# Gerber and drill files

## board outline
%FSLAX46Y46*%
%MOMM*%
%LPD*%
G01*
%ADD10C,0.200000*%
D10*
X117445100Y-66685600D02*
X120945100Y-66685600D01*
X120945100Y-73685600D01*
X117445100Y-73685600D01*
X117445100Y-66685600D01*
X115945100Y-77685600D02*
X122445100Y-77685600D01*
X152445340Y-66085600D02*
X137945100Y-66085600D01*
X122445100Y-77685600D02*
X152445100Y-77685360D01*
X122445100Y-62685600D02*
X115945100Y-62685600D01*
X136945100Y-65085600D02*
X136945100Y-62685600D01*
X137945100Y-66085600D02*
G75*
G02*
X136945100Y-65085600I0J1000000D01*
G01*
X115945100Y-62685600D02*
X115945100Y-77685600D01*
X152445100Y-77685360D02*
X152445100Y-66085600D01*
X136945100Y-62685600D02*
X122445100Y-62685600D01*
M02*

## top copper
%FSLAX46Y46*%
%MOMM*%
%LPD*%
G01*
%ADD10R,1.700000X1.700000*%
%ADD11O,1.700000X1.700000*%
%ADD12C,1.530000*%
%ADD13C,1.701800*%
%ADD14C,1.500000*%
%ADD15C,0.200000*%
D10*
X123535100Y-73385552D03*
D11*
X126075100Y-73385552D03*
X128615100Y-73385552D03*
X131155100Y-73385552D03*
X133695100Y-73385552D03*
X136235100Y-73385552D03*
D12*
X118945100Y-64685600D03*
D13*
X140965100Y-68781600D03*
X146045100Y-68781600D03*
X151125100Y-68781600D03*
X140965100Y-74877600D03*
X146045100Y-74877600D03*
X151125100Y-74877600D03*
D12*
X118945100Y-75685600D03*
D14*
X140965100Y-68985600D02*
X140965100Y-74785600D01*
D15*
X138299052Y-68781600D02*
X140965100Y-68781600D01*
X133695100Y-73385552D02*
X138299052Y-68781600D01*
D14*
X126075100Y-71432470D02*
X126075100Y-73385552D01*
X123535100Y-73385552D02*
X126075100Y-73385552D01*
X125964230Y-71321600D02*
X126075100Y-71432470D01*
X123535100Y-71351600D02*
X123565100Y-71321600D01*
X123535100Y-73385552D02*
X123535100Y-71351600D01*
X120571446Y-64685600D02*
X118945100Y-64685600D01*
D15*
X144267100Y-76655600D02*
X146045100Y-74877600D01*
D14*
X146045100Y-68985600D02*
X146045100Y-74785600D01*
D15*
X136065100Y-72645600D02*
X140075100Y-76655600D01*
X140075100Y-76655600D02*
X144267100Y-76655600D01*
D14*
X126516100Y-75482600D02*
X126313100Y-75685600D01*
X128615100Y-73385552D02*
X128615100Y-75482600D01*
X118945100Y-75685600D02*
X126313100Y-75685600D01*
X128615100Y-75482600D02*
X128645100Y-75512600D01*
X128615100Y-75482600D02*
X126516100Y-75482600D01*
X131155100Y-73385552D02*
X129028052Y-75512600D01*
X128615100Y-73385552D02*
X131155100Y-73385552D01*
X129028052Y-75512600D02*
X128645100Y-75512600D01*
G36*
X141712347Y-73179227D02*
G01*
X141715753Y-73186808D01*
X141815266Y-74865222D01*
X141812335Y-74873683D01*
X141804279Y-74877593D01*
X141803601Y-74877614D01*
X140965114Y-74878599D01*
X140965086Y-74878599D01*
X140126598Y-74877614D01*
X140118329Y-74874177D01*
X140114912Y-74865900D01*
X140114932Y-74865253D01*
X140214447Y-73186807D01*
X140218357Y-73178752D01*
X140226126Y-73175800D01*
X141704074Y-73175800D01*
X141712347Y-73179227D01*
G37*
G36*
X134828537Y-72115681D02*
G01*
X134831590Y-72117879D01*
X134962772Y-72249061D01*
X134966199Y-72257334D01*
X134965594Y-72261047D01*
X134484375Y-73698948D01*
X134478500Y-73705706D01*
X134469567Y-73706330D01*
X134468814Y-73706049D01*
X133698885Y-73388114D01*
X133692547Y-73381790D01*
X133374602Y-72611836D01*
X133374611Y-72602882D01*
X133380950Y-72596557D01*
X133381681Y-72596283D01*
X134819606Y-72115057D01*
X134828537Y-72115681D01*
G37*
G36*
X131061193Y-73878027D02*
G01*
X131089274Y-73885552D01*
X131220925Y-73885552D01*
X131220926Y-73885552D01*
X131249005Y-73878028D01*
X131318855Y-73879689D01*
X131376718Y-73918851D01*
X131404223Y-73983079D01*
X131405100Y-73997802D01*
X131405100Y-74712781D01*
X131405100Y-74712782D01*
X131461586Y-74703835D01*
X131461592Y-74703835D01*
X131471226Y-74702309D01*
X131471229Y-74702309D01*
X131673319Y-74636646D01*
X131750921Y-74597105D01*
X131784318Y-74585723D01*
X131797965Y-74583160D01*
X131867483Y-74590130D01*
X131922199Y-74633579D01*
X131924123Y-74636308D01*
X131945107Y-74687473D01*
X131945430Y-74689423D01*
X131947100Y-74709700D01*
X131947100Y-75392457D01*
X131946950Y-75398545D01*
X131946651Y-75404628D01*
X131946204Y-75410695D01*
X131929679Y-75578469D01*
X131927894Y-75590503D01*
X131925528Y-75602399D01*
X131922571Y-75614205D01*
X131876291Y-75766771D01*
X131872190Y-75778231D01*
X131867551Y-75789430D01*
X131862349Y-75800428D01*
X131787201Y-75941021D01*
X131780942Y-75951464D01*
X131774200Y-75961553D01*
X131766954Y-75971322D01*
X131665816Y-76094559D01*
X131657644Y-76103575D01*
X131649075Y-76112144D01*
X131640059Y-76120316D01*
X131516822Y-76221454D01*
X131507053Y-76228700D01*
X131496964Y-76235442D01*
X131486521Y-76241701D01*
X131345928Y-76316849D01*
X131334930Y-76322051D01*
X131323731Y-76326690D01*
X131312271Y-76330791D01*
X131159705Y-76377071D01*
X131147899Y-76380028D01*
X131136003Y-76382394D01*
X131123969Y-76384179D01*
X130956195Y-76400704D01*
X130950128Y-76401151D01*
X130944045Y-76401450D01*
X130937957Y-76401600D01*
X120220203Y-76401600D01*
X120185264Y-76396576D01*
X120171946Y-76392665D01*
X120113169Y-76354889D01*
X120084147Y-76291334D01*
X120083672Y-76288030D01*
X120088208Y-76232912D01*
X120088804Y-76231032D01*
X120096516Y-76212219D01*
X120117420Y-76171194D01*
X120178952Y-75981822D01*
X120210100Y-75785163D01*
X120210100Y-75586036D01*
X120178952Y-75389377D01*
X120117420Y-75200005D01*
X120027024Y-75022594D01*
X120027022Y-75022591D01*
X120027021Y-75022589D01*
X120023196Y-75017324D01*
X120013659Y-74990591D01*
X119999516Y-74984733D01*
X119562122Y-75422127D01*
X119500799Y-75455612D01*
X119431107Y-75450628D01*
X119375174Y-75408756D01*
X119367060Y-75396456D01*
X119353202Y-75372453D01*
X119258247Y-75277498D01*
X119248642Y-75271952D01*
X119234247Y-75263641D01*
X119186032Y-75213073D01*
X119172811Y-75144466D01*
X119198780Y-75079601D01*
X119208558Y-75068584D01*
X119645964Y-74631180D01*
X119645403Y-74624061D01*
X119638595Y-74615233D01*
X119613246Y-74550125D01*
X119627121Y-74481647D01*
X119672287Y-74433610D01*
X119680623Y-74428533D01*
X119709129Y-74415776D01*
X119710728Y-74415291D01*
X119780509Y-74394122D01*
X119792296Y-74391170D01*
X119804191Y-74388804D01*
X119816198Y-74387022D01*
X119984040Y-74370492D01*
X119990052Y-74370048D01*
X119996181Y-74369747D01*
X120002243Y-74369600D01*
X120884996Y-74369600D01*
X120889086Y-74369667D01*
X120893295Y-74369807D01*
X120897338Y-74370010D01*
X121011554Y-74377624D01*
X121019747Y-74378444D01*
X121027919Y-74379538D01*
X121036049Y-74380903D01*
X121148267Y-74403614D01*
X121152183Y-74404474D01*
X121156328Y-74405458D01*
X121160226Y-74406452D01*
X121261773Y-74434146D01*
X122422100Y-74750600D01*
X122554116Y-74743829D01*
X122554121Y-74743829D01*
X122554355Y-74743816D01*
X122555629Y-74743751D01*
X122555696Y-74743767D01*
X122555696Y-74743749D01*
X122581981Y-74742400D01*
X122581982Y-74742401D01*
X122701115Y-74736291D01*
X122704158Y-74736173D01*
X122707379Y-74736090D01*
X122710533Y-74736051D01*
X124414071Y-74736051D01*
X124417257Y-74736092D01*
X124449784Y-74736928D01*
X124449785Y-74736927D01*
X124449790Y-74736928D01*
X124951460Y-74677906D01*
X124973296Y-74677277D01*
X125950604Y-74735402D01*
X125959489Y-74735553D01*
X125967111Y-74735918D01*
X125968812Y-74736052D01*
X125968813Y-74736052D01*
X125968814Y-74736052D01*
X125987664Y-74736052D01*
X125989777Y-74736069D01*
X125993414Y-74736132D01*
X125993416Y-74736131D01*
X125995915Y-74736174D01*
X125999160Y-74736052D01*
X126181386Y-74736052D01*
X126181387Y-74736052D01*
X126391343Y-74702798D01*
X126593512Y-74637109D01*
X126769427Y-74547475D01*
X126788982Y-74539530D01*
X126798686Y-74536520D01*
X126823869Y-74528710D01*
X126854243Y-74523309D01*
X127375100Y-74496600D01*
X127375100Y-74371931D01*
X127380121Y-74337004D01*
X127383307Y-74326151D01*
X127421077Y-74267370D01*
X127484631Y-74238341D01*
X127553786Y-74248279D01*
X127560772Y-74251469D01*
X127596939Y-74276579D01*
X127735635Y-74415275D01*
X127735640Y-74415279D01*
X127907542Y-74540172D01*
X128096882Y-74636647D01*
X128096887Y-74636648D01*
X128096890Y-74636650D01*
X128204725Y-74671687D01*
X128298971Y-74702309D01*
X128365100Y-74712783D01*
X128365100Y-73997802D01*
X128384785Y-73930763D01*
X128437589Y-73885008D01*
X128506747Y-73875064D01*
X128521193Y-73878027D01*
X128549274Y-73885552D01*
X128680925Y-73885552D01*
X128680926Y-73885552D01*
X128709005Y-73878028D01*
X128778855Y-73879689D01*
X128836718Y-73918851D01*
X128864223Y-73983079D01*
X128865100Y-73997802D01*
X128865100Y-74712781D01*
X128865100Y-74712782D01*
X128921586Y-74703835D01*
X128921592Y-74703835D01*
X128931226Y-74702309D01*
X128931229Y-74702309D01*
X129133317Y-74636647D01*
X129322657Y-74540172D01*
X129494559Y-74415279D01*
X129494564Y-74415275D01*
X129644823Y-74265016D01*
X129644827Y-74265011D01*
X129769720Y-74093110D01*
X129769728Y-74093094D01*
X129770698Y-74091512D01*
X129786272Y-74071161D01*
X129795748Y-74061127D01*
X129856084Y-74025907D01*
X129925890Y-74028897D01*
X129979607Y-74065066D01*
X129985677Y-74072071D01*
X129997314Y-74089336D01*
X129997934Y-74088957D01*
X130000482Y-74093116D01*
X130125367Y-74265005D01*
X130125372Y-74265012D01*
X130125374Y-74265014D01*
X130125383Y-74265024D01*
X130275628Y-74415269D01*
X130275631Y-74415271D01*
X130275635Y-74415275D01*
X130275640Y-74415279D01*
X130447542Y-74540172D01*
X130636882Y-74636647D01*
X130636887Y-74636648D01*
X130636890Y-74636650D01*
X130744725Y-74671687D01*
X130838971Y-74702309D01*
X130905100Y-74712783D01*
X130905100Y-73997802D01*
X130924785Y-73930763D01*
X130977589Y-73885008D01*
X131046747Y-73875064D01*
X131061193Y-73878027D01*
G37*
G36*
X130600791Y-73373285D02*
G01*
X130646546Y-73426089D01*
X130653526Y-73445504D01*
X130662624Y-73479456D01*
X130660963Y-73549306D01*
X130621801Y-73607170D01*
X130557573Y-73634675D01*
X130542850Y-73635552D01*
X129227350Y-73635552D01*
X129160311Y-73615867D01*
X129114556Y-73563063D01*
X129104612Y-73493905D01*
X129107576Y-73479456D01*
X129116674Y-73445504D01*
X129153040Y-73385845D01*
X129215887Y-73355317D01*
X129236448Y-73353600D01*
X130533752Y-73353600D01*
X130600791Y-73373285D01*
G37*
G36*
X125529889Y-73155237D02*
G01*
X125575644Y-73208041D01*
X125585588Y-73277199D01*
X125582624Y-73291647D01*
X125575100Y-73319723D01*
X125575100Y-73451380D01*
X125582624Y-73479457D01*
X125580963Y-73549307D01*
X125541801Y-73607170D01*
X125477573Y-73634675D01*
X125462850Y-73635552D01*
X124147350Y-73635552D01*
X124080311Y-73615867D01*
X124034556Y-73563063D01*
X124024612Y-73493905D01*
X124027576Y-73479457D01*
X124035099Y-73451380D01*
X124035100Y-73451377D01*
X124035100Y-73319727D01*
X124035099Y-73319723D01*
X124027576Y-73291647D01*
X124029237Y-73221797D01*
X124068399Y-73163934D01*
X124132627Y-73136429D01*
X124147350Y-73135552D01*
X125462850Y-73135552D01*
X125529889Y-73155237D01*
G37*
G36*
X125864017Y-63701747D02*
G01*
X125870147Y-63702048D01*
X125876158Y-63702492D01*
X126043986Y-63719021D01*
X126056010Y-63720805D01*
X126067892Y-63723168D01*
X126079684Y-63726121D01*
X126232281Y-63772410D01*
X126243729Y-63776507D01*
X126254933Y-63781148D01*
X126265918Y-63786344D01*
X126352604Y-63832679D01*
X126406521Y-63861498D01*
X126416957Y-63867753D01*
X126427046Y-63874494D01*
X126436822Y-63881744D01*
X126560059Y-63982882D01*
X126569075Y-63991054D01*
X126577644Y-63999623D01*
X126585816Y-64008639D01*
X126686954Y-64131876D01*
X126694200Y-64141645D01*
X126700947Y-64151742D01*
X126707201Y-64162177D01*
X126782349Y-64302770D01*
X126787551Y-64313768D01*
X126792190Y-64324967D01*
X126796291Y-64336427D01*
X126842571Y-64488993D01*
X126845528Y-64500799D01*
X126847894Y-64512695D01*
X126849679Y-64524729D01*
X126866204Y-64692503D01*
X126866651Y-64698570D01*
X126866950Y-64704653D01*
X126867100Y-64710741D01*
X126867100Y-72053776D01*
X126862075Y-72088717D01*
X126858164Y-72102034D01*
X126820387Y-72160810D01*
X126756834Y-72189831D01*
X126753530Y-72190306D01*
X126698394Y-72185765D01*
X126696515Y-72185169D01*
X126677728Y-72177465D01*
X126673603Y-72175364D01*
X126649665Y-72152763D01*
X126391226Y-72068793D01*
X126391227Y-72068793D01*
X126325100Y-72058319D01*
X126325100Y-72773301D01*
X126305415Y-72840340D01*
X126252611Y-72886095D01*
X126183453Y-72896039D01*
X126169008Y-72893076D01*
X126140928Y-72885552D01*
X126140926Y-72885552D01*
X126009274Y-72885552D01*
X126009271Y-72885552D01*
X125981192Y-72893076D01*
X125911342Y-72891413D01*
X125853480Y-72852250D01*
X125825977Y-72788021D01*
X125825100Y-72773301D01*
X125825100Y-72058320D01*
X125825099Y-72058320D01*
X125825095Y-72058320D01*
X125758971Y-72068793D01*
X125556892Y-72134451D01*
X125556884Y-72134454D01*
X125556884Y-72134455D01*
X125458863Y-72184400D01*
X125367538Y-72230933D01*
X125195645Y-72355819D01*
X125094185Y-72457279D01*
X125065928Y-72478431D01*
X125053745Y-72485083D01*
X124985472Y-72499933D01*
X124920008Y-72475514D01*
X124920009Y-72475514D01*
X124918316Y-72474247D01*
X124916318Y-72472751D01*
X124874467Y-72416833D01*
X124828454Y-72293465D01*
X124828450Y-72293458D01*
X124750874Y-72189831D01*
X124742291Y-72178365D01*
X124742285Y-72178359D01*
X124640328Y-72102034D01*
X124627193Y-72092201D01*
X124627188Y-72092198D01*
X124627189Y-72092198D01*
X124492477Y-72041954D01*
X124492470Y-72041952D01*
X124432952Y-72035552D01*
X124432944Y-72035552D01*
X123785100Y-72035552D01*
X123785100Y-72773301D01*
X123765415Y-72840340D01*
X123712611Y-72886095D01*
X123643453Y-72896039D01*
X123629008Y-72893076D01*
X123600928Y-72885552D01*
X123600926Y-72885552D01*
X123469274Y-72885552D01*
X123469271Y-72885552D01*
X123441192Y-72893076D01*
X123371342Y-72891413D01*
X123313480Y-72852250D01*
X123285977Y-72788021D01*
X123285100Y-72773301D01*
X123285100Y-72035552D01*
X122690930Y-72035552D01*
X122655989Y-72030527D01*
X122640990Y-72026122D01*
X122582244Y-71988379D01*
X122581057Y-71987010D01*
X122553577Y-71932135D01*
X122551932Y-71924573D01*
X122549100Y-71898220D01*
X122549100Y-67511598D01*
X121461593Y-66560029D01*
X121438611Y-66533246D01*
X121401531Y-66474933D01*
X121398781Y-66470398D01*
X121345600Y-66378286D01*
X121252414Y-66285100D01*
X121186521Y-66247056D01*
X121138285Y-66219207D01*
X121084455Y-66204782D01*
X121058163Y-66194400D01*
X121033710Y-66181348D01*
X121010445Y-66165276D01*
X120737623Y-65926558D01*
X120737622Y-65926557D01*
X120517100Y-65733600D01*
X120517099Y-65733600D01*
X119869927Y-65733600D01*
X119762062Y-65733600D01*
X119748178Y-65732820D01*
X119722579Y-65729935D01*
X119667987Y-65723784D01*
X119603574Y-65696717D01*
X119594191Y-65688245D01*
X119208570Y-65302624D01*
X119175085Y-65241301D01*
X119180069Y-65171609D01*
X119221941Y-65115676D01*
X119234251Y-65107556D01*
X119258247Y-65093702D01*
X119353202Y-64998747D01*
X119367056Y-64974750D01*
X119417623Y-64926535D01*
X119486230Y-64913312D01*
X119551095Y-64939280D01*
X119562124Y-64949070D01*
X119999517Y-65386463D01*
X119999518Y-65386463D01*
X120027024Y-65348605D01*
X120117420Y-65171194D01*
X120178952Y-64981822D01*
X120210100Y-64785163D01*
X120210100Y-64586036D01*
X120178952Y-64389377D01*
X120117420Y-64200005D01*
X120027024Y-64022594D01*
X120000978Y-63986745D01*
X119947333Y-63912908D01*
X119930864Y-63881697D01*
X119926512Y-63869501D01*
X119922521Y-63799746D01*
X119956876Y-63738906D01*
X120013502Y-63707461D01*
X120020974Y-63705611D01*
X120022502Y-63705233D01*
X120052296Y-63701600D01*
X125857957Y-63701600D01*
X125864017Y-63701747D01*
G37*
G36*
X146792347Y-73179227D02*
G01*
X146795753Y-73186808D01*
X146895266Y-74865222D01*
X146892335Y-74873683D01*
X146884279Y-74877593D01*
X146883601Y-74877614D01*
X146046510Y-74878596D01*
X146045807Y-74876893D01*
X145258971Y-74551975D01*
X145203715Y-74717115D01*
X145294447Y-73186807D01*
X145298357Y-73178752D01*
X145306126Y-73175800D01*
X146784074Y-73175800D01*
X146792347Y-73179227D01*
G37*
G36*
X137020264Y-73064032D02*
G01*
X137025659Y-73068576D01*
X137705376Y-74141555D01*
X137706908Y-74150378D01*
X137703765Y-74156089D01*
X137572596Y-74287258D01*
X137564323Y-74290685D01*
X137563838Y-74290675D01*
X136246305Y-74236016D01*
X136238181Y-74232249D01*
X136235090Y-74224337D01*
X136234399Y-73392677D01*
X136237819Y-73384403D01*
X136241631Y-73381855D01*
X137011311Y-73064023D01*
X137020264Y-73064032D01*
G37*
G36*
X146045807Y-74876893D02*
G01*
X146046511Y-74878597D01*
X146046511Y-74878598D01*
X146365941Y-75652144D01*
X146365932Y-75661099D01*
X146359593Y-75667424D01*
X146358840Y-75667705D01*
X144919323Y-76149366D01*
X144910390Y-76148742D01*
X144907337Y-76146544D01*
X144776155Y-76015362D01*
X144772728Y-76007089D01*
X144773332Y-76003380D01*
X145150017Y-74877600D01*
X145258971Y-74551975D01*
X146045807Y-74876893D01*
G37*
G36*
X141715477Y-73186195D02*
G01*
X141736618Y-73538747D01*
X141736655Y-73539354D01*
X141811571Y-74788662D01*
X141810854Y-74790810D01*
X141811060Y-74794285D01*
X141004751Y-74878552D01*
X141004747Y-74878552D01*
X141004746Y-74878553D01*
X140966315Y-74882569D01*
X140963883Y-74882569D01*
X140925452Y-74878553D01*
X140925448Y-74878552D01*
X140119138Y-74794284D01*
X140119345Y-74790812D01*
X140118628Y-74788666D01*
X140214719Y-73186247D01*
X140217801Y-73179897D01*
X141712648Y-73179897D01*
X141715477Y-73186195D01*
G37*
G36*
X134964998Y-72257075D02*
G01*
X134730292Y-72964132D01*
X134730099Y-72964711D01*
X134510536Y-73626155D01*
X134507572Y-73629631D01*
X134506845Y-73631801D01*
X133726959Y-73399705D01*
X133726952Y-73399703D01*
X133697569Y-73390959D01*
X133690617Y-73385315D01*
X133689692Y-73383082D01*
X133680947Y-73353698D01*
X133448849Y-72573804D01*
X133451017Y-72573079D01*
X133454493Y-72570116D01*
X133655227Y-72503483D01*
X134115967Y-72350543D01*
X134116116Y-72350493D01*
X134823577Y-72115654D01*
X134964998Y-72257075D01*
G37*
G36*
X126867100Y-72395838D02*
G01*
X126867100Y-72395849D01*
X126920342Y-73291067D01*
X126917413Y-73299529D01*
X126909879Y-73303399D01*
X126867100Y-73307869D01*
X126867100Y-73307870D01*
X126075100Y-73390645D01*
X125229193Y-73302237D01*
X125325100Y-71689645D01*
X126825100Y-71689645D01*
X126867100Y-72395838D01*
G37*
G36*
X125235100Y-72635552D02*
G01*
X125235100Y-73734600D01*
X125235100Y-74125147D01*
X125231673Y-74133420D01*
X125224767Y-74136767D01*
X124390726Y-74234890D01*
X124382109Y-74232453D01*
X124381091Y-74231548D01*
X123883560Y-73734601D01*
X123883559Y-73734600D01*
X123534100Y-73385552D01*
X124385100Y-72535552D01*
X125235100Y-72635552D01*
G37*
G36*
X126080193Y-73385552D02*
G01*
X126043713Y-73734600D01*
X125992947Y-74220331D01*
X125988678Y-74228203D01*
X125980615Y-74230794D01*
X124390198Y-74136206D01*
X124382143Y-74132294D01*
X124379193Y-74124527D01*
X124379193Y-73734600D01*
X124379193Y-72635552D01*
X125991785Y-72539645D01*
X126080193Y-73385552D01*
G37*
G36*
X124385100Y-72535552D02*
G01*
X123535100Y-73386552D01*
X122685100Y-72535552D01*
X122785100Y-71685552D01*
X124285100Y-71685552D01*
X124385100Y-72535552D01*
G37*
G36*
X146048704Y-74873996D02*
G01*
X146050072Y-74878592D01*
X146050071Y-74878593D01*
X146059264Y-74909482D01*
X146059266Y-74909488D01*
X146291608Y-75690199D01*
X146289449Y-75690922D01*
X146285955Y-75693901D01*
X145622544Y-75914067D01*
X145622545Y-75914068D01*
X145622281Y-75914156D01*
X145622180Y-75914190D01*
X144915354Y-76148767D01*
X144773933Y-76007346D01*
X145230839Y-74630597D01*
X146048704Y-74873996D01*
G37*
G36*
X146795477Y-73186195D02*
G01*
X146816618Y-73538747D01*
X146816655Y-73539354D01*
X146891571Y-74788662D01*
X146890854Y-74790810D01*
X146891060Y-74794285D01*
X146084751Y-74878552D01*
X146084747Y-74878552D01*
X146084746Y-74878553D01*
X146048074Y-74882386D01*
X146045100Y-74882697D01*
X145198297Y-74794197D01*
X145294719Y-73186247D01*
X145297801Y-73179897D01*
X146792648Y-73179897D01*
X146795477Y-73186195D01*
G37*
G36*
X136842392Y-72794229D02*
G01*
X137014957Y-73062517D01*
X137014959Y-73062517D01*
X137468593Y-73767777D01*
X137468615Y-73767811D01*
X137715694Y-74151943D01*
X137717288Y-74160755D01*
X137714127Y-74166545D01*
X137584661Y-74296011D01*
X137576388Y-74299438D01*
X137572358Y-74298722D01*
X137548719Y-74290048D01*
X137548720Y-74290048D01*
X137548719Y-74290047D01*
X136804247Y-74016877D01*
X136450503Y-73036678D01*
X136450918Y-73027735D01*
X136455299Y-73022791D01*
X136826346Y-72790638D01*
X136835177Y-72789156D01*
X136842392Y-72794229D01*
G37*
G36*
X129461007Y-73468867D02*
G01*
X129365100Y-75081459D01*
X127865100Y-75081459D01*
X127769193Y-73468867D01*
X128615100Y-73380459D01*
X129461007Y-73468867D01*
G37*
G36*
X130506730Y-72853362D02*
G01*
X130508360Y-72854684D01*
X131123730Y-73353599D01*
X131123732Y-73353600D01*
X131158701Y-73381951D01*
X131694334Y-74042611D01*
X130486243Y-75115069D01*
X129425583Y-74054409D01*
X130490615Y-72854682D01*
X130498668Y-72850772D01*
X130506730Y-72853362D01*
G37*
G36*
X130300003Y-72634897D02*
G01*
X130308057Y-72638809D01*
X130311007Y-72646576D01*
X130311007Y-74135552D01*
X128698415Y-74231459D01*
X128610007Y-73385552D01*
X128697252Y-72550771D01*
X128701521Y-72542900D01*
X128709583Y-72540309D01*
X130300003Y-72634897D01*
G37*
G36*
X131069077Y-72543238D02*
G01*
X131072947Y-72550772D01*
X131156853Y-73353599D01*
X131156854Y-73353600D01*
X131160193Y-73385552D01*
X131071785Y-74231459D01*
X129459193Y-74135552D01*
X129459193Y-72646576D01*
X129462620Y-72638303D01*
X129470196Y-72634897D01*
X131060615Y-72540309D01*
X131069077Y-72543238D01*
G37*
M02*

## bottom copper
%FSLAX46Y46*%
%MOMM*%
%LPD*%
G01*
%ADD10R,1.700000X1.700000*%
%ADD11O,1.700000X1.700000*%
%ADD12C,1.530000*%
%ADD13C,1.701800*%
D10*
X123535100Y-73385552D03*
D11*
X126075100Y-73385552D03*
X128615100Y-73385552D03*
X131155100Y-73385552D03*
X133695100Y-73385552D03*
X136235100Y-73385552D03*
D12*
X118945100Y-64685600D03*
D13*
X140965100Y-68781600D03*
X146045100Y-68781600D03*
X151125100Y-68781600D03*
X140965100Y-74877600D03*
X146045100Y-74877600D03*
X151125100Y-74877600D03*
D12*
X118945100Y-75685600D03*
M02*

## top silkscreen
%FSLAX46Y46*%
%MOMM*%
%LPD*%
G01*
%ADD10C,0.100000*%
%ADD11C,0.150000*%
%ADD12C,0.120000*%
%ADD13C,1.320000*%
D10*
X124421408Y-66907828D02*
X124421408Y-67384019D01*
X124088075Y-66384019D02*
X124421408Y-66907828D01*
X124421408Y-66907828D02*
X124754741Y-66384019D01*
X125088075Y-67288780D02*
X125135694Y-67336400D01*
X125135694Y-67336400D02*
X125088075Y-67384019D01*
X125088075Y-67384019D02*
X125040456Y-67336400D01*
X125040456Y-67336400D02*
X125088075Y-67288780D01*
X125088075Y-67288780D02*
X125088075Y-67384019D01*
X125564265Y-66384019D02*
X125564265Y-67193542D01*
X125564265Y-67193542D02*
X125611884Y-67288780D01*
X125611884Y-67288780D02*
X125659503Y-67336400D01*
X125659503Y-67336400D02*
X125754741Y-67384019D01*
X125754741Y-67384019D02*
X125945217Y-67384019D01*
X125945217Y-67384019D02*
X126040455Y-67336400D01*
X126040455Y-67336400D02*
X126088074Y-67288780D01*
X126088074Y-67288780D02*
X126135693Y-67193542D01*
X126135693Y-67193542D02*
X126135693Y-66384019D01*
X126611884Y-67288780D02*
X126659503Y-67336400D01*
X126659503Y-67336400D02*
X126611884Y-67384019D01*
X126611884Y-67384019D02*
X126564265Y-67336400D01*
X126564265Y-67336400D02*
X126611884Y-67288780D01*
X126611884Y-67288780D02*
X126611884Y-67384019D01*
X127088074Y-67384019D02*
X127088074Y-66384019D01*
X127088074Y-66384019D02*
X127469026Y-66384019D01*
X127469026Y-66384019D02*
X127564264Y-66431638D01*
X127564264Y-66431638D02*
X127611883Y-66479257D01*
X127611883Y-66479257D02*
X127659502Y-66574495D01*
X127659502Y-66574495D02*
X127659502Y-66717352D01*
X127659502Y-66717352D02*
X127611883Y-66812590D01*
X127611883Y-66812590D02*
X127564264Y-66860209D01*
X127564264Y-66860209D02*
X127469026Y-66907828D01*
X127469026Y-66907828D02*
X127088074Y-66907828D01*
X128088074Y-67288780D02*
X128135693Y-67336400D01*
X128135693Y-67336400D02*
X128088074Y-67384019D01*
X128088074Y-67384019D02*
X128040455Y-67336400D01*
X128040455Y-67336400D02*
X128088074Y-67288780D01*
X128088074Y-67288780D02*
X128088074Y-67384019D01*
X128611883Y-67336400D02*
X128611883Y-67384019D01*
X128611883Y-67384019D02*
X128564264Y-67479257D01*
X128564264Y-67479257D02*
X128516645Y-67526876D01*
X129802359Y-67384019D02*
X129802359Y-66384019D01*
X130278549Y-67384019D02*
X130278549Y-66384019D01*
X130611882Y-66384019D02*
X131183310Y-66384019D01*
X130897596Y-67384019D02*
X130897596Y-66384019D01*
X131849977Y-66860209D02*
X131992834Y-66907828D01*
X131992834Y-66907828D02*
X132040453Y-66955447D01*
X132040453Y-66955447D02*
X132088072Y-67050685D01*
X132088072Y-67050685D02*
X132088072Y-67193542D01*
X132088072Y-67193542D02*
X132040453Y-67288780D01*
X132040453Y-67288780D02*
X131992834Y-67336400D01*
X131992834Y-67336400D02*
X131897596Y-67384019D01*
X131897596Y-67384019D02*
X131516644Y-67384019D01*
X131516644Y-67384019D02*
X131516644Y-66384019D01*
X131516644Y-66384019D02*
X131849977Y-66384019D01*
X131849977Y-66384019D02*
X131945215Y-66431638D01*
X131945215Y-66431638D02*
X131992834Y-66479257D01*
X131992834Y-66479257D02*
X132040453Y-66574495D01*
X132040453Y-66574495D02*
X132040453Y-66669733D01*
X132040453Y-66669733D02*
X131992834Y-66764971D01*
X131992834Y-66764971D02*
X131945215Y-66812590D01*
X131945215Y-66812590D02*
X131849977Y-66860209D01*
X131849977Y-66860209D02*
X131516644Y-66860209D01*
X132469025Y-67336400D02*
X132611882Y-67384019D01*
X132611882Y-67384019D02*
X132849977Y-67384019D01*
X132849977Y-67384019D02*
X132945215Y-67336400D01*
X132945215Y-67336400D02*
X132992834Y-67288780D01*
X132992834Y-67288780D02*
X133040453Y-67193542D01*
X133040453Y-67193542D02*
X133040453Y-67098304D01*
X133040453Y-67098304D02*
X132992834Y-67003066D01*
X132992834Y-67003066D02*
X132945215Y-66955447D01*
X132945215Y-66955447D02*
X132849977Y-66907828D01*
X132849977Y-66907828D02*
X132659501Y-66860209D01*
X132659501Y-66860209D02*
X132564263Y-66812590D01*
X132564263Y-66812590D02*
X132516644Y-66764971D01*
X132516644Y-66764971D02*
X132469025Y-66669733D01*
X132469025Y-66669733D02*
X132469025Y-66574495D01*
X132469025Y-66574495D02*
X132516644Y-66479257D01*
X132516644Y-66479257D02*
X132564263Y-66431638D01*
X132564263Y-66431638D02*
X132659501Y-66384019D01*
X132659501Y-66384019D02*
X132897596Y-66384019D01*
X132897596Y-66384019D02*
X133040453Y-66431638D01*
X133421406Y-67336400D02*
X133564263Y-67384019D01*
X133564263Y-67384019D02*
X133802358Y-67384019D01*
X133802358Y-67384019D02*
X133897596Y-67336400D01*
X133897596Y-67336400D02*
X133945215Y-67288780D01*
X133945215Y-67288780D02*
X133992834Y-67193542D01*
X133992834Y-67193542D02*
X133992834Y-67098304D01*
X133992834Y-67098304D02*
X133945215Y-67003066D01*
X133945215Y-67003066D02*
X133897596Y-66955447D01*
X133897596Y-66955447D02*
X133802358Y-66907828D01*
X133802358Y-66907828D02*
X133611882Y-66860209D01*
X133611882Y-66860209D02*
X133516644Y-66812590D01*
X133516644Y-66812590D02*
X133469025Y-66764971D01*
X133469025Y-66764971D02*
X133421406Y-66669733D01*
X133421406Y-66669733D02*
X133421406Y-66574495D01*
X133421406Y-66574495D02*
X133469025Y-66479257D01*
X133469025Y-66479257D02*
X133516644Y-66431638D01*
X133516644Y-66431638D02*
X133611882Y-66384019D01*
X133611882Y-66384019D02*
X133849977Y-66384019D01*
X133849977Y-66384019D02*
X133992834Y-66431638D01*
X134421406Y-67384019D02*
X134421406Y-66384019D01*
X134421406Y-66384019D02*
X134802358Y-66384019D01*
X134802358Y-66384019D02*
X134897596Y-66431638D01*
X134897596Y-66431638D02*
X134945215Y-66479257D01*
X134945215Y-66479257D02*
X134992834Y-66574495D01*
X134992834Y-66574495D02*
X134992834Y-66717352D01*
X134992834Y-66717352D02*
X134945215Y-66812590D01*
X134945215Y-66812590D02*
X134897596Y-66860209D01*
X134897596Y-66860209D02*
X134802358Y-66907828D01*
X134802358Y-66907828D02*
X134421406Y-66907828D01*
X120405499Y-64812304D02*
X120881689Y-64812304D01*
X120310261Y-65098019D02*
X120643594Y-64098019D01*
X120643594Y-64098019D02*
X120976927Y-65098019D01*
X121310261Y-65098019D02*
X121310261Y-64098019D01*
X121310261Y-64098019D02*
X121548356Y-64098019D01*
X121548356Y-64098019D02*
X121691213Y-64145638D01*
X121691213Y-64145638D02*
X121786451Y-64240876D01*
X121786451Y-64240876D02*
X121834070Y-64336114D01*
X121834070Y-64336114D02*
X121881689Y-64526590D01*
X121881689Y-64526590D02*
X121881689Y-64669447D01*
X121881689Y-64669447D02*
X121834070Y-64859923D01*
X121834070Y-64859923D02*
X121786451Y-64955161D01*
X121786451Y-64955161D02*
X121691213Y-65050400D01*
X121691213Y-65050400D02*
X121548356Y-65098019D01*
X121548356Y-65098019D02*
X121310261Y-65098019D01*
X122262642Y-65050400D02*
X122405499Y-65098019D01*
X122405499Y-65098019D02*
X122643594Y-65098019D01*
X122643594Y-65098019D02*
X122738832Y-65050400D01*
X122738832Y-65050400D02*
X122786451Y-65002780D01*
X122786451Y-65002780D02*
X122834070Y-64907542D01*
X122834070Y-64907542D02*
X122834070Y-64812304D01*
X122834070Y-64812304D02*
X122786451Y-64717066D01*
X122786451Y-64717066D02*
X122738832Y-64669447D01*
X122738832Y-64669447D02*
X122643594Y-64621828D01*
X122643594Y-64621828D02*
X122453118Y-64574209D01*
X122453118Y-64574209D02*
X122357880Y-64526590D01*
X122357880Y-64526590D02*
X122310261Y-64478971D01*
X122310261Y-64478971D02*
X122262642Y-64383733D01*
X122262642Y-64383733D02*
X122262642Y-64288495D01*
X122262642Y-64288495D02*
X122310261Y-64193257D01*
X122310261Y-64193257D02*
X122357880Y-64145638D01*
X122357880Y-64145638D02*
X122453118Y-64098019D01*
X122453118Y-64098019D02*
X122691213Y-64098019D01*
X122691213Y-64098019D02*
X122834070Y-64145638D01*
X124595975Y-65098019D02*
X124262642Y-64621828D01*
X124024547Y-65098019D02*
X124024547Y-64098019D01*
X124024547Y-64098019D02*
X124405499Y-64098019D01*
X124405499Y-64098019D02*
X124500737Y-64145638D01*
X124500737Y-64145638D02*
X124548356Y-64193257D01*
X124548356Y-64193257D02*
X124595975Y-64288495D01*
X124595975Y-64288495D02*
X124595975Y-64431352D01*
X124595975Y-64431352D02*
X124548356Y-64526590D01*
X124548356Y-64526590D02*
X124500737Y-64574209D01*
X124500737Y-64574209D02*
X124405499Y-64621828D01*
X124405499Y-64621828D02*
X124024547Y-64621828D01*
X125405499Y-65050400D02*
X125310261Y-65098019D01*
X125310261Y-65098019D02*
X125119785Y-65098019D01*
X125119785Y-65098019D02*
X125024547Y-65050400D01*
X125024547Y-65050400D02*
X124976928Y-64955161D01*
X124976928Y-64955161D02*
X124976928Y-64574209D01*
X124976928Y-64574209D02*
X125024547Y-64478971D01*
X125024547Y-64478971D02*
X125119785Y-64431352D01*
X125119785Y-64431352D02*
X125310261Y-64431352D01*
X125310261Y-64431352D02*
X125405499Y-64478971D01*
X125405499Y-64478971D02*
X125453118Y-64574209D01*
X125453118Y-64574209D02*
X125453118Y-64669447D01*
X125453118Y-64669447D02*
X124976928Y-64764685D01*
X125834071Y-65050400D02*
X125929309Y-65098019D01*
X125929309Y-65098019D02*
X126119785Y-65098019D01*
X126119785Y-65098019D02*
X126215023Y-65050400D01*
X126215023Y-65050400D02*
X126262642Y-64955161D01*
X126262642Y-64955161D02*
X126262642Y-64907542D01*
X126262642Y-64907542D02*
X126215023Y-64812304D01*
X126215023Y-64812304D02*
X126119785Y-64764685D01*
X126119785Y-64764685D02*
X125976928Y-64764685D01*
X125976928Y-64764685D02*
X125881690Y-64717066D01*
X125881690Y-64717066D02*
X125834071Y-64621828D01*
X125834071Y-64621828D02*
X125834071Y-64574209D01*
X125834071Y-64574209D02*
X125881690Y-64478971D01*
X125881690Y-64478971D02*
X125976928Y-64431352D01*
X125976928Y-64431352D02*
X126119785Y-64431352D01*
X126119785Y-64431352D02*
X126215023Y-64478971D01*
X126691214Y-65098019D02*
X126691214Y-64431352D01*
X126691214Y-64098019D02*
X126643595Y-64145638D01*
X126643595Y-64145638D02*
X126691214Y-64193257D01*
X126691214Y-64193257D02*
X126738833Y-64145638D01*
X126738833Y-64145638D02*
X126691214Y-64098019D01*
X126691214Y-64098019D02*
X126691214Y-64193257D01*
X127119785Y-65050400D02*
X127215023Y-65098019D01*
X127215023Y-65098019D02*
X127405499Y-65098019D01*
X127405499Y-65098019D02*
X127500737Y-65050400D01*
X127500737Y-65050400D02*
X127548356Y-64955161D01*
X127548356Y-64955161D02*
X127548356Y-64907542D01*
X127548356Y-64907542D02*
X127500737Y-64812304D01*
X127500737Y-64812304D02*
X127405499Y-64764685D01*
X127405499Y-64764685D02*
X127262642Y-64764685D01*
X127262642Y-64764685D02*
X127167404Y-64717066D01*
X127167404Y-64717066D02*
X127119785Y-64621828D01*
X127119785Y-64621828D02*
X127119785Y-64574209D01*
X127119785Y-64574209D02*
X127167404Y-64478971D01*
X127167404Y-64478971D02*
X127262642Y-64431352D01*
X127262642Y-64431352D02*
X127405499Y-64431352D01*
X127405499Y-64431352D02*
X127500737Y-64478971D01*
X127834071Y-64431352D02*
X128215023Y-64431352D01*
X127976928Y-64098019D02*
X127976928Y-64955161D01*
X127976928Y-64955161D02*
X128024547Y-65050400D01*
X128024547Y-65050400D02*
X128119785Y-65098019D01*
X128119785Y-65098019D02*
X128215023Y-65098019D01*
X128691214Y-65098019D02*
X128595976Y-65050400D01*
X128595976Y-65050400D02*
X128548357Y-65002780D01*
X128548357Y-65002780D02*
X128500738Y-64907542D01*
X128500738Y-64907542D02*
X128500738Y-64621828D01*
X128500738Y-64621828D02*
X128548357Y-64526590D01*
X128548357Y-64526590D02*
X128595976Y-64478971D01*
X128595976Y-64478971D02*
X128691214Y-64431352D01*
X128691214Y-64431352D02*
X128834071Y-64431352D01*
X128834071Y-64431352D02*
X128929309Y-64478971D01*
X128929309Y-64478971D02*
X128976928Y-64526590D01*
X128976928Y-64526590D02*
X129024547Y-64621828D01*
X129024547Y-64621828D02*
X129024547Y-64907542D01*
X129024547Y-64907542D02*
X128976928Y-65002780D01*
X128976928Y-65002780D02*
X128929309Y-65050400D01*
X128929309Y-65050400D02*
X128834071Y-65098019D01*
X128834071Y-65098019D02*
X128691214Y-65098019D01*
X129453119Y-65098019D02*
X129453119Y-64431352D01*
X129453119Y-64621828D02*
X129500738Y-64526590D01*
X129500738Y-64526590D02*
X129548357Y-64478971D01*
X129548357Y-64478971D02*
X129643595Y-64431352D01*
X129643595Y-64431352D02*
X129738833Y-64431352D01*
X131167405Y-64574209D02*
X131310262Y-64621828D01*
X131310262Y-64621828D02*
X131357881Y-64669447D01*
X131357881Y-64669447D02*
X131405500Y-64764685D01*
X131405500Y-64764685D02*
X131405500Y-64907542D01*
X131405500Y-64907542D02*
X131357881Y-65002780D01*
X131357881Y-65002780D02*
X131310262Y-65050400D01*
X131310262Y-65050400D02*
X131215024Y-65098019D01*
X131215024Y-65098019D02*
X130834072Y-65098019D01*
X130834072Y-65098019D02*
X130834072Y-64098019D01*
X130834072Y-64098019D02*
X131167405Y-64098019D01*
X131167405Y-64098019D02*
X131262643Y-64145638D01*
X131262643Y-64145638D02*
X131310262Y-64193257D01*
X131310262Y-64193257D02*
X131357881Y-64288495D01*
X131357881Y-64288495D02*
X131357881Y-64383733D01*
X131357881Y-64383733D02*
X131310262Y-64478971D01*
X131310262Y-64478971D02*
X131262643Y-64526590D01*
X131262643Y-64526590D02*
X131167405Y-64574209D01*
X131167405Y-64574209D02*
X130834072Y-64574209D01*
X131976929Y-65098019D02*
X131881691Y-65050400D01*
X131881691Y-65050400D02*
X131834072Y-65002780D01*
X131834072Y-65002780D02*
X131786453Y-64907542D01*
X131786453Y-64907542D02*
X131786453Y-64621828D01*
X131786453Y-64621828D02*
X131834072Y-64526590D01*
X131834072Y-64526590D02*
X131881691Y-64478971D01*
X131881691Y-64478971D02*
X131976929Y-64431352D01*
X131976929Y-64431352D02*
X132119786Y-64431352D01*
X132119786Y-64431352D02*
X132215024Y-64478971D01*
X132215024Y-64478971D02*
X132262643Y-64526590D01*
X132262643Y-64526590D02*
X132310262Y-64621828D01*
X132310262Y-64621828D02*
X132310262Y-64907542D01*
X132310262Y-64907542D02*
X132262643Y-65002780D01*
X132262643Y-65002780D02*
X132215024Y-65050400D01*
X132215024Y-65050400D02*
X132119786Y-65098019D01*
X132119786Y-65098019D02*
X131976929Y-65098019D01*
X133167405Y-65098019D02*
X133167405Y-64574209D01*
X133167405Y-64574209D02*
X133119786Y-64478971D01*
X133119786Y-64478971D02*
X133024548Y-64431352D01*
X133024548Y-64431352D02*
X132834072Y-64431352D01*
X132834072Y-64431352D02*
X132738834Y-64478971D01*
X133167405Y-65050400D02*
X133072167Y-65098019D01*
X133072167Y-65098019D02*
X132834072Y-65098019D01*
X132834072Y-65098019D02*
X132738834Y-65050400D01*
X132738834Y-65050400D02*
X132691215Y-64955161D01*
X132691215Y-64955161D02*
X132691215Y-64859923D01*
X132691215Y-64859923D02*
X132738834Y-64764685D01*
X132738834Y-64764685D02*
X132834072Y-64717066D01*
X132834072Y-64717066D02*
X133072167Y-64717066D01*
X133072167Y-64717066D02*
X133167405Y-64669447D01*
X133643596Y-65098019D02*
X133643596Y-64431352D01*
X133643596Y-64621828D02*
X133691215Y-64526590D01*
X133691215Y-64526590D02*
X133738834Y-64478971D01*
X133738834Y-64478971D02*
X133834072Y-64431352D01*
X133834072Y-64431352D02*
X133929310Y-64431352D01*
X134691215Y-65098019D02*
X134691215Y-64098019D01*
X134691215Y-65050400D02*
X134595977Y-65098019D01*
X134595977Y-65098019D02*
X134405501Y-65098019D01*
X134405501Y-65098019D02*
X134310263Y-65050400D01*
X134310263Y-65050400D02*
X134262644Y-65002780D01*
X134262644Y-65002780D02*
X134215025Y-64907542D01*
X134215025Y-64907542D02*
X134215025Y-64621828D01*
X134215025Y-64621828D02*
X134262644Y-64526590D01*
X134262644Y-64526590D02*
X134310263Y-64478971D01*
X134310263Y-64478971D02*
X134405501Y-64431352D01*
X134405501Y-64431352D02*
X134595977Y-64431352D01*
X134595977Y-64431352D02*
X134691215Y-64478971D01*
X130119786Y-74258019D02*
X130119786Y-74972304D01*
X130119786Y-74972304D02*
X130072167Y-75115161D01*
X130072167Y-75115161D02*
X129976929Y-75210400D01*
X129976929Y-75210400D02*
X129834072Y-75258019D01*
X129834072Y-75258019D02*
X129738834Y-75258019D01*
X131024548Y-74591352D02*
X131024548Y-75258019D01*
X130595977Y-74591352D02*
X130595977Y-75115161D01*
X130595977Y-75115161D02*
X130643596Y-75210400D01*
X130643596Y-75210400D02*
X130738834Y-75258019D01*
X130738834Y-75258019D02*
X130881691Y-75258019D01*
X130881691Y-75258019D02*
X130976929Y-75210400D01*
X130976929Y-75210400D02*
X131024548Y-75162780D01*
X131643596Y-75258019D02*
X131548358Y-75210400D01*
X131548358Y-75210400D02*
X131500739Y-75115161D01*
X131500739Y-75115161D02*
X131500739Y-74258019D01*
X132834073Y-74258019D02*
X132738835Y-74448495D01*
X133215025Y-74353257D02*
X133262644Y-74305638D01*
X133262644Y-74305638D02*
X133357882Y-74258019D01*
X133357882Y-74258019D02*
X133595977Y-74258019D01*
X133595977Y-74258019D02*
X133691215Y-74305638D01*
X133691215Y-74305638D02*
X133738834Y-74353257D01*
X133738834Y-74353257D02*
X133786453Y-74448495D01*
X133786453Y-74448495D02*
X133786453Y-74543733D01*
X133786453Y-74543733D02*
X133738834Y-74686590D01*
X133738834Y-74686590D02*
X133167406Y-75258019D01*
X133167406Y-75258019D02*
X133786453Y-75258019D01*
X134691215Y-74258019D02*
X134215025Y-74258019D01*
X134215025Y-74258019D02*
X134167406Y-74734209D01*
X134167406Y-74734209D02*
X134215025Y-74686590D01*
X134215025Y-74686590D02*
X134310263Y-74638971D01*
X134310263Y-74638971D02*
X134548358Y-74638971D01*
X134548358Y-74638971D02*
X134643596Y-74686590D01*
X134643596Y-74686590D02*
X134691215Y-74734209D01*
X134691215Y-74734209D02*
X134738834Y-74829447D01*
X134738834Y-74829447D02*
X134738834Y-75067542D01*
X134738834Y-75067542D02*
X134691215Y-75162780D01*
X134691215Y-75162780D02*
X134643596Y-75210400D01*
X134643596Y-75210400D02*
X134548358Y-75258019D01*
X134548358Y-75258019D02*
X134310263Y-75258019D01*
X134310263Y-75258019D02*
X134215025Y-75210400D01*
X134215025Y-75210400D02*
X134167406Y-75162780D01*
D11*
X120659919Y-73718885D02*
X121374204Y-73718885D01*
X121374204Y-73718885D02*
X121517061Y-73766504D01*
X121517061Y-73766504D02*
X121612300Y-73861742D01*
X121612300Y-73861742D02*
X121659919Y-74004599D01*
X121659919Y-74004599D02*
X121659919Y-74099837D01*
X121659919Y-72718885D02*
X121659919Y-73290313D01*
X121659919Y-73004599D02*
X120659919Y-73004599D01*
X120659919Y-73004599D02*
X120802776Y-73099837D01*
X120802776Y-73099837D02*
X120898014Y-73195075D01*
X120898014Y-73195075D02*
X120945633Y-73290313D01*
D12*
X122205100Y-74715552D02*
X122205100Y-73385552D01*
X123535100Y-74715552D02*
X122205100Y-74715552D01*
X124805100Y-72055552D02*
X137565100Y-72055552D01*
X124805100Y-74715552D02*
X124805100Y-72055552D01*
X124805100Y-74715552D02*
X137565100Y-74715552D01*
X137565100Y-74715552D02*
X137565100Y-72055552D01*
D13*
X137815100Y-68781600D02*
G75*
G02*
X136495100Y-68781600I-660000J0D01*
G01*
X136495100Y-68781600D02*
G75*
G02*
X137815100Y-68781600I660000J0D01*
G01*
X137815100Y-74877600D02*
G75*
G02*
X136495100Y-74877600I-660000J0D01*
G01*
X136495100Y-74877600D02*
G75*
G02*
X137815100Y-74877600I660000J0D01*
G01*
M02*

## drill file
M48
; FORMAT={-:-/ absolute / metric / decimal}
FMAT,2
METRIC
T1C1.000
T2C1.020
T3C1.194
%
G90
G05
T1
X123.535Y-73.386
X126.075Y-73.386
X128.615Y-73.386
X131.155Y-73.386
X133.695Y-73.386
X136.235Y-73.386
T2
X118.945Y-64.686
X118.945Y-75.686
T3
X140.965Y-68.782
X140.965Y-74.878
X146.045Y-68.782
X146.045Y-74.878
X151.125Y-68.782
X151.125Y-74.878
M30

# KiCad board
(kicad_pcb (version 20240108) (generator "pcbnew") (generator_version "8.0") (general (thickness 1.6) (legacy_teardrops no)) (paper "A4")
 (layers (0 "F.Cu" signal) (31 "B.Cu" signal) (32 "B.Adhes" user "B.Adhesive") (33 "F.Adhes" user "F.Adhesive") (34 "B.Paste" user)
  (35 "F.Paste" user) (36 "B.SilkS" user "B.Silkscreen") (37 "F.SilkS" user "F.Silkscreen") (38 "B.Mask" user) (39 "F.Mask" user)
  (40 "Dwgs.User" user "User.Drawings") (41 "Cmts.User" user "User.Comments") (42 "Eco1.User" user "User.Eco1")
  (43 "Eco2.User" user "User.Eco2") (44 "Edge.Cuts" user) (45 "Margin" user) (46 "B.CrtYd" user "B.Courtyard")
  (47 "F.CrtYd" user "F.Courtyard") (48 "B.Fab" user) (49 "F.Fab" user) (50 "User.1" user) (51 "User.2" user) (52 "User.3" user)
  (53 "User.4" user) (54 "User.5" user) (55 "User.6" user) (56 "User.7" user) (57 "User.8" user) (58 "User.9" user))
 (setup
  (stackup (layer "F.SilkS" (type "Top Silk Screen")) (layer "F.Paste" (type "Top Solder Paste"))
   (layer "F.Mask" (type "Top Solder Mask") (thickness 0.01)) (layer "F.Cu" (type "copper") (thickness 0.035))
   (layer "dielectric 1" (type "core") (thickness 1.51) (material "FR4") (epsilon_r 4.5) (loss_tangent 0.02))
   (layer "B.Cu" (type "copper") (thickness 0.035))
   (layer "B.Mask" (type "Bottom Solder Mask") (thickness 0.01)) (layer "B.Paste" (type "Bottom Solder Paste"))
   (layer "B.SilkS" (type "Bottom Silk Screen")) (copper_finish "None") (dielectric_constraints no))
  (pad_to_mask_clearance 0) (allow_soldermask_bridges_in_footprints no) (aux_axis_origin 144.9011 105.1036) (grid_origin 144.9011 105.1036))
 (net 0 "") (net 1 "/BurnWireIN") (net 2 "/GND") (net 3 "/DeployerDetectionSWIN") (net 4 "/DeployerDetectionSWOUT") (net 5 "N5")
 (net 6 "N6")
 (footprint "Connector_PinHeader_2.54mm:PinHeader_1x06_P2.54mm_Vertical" (layer "F.Cu") (at 123.5351 73.385552 90)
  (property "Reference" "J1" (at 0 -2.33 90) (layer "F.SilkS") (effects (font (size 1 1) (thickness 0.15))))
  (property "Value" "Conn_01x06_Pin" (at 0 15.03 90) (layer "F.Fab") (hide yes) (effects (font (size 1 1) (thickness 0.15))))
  (fp_line (start -1.33 -1.33) (end 0 -1.33) (stroke (width 0.12) (type solid)) (layer "F.SilkS"))
  (fp_line (start -1.33 0) (end -1.33 -1.33) (stroke (width 0.12) (type solid)) (layer "F.SilkS"))
  (fp_line (start 1.33 1.27) (end 1.33 14.03) (stroke (width 0.12) (type solid)) (layer "F.SilkS"))
  (fp_line (start -1.33 1.27) (end 1.33 1.27) (stroke (width 0.12) (type solid)) (layer "F.SilkS"))
  (fp_line (start -1.33 1.27) (end -1.33 14.03) (stroke (width 0.12) (type solid)) (layer "F.SilkS"))
  (fp_line (start -1.33 14.03) (end 1.33 14.03) (stroke (width 0.12) (type solid)) (layer "F.SilkS"))
  (pad "1" thru_hole rect (at 0 0 90) (size 1.7 1.7) (drill 1) (layers "*.Cu" "*.Mask") (remove_unused_layers no) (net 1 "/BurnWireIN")
   (teardrops (best_length_ratio 0.5) (max_length 1) (best_width_ratio 1) (max_width 2) (curve_points 0) (filter_ratio 0.9) (enabled yes)
    (allow_two_segments yes) (prefer_zone_connections yes)))
  (pad "2" thru_hole oval (at 0 2.54 90) (size 1.7 1.7) (drill 1) (layers "*.Cu" "*.Mask") (remove_unused_layers no) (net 1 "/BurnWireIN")
   (teardrops (best_length_ratio 0.5) (max_length 1) (best_width_ratio 1) (max_width 2) (curve_points 0) (filter_ratio 0.9) (enabled yes)
    (allow_two_segments yes) (prefer_zone_connections yes)))
  (pad "3" thru_hole oval (at 0 5.08 90) (size 1.7 1.7) (drill 1) (layers "*.Cu" "*.Mask") (remove_unused_layers no) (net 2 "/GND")
   (teardrops (best_length_ratio 0.5) (max_length 1) (best_width_ratio 1) (max_width 2) (curve_points 0) (filter_ratio 0.9) (enabled yes)
    (allow_two_segments yes) (prefer_zone_connections yes)))
  (pad "4" thru_hole oval (at 0 7.62 90) (size 1.7 1.7) (drill 1) (layers "*.Cu" "*.Mask") (remove_unused_layers no) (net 2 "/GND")
   (teardrops (best_length_ratio 0.5) (max_length 1) (best_width_ratio 1) (max_width 2) (curve_points 0) (filter_ratio 0.9) (enabled yes)
    (allow_two_segments yes) (prefer_zone_connections yes)))
  (pad "5" thru_hole oval (at 0 10.16 90) (size 1.7 1.7) (drill 1) (layers "*.Cu" "*.Mask") (remove_unused_layers no)
   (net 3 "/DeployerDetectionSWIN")
   (teardrops (best_length_ratio 0.5) (max_length 1) (best_width_ratio 1) (max_width 2) (curve_points 0) (filter_ratio 0.9) (enabled yes)
    (allow_two_segments yes) (prefer_zone_connections yes)))
  (pad "6" thru_hole oval (at 0 12.7 90) (size 1.7 1.7) (drill 1) (layers "*.Cu" "*.Mask") (remove_unused_layers no)
   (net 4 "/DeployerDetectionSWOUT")
   (teardrops (best_length_ratio 0.5) (max_length 1) (best_width_ratio 1) (max_width 2) (curve_points 0) (filter_ratio 0.9) (enabled yes)
    (allow_two_segments yes) (prefer_zone_connections yes))))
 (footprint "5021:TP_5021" (layer "B.Cu") (at 118.9451 64.6856 -90)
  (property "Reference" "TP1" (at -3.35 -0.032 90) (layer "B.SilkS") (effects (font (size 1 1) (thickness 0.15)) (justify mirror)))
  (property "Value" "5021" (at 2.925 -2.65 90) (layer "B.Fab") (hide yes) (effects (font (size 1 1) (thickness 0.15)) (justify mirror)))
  (pad "TP" thru_hole circle (at 0 0 270) (size 1.53 1.53) (drill 1.02) (layers "*.Cu" "*.Mask") (remove_unused_layers no)
   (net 1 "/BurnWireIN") (solder_mask_margin 0.102)
   (teardrops (best_length_ratio 0.5) (max_length 1) (best_width_ratio 1) (max_width 2) (curve_points 0) (filter_ratio 0.9) (enabled yes)
    (allow_two_segments yes) (prefer_zone_connections yes))))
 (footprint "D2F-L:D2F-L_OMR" (layer "B.Cu") (at 140.9651 68.7816)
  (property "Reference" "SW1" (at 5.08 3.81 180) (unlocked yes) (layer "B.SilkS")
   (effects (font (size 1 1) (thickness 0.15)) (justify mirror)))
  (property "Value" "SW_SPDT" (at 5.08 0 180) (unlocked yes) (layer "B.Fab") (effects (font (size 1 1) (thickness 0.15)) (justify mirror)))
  (fp_circle (center -3.81 0) (end -2.54 0) (stroke (width 0.1) (type solid)) (fill solid) (layer "F.SilkS"))
  (pad "1" thru_hole circle (at 0 0) (size 1.7018 1.7018) (drill 1.1938) (layers "*.Cu" "*.Mask") (remove_unused_layers no)
   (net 3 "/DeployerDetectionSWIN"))
  (pad "2" thru_hole circle (at 5.08 0) (size 1.7018 1.7018) (drill 1.1938) (layers "*.Cu" "*.Mask") (remove_unused_layers no)
   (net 4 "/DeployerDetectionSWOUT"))
  (pad "3" thru_hole circle (at 10.16 0) (size 1.7018 1.7018) (drill 1.1938) (layers "*.Cu" "*.Mask") (remove_unused_layers no) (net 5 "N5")))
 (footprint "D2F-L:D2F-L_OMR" (layer "B.Cu") (at 140.9651 74.8776)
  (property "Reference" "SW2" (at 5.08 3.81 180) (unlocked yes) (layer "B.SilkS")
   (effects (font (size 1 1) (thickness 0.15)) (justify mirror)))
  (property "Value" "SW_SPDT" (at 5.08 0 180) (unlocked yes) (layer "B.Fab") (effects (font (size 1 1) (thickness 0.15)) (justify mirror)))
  (fp_circle (center -3.81 0) (end -2.54 0) (stroke (width 0.1) (type solid)) (fill solid) (layer "F.SilkS"))
  (pad "1" thru_hole circle (at 0 0) (size 1.7018 1.7018) (drill 1.1938) (layers "*.Cu" "*.Mask") (remove_unused_layers no)
   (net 3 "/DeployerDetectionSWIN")
   (teardrops (best_length_ratio 0.5) (max_length 1) (best_width_ratio 1) (max_width 2) (curve_points 0) (filter_ratio 0.9) (enabled yes)
    (allow_two_segments yes) (prefer_zone_connections yes)))
  (pad "2" thru_hole circle (at 5.08 0) (size 1.7018 1.7018) (drill 1.1938) (layers "*.Cu" "*.Mask") (remove_unused_layers no)
   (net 4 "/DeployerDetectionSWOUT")
   (teardrops (best_length_ratio 0.5) (max_length 1) (best_width_ratio 1) (max_width 2) (curve_points 0) (filter_ratio 0.9) (enabled yes)
    (allow_two_segments yes) (prefer_zone_connections yes)))
  (pad "3" thru_hole circle (at 10.16 0) (size 1.7018 1.7018) (drill 1.1938) (layers "*.Cu" "*.Mask") (remove_unused_layers no) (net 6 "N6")
   (teardrops (best_length_ratio 0.5) (max_length 1) (best_width_ratio 1) (max_width 2) (curve_points 0) (filter_ratio 0.9) (enabled yes)
    (allow_two_segments yes) (prefer_zone_connections yes))))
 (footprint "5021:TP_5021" (layer "B.Cu") (at 118.9451 75.6856 -90)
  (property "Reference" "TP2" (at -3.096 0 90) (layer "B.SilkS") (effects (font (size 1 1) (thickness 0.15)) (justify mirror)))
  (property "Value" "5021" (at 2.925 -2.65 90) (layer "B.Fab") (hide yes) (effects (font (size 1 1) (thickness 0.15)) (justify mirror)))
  (pad "TP" thru_hole circle (at 0 0 270) (size 1.53 1.53) (drill 1.02) (layers "*.Cu" "*.Mask") (remove_unused_layers no) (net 2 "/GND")
   (solder_mask_margin 0.102)
   (teardrops (best_length_ratio 0.5) (max_length 1) (best_width_ratio 1) (max_width 2) (curve_points 0) (filter_ratio 0.9) (enabled yes)
    (allow_two_segments yes) (prefer_zone_connections yes))))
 (gr_rect (start 117.4451 66.6856) (end 120.9451 73.6856) (stroke (width 0.2) (type default)) (fill none) (layer "Edge.Cuts"))
 (gr_line (start 115.9451 77.6856) (end 122.4451 77.6856) (locked yes) (stroke (width 0.2) (type default)) (layer "Edge.Cuts"))
 (gr_line (start 152.44534 66.0856) (end 137.9451 66.0856) (locked yes) (stroke (width 0.2) (type default)) (layer "Edge.Cuts"))
 (gr_line (start 122.4451 77.6856) (end 152.4451 77.68536) (locked yes) (stroke (width 0.2) (type default)) (layer "Edge.Cuts"))
 (gr_line (start 122.4451 62.6856) (end 115.9451 62.6856) (locked yes) (stroke (width 0.2) (type default)) (layer "Edge.Cuts"))
 (gr_line (start 136.9451 65.0856) (end 136.9451 62.6856) (locked yes) (stroke (width 0.2) (type default)) (layer "Edge.Cuts"))
 (gr_arc (start 137.9451 66.0856) (mid 137.237993 65.792707) (end 136.9451 65.0856) (locked yes) (stroke (width 0.2) (type default))
  (layer "Edge.Cuts"))
 (gr_line (start 115.9451 62.6856) (end 115.9451 77.6856) (locked yes) (stroke (width 0.2) (type default)) (layer "Edge.Cuts"))
 (gr_line (start 152.4451 77.68536) (end 152.4451 66.0856) (locked yes) (stroke (width 0.2) (type default)) (layer "Edge.Cuts"))
 (gr_line (start 136.9451 62.6856) (end 122.4451 62.6856) (locked yes) (stroke (width 0.2) (type default)) (layer "Edge.Cuts"))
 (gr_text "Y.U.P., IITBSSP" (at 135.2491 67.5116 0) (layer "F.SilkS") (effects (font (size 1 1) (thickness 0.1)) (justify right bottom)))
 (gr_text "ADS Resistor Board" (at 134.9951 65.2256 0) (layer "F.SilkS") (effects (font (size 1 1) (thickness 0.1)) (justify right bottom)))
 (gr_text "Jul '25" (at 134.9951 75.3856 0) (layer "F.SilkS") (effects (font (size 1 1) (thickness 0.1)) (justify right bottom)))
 (segment (start 140.9651 68.9856) (end 140.9651 74.7856) (width 1.5) (layer "F.Cu") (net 3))
 (segment (start 138.299052 68.7816) (end 140.9651 68.7816) (width 0.2) (layer "F.Cu") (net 3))
 (segment (start 133.6951 73.385552) (end 138.299052 68.7816) (width 0.2) (layer "F.Cu") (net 3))
 (segment (start 126.0751 71.43247) (end 126.0751 73.385552) (width 1.5) (layer "F.Cu") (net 1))
 (segment (start 123.5351 73.385552) (end 126.0751 73.385552) (width 1.5) (layer "F.Cu") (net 1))
 (segment (start 125.96423 71.3216) (end 126.0751 71.43247) (width 1.5) (layer "F.Cu") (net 1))
 (segment (start 123.5351 71.3516) (end 123.5651 71.3216) (width 1.5) (layer "F.Cu") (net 1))
 (segment (start 123.5351 73.385552) (end 123.5351 71.3516) (width 1.5) (layer "F.Cu") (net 1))
 (segment (start 120.571446 64.6856) (end 118.9451 64.6856) (width 1.5) (layer "F.Cu") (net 1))
 (segment (start 144.2671 76.6556) (end 146.0451 74.8776) (width 0.2) (layer "F.Cu") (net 4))
 (segment (start 146.0451 68.9856) (end 146.0451 74.7856) (width 1.5) (layer "F.Cu") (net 4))
 (segment (start 136.0651 72.6456) (end 140.0751 76.6556) (width 0.2) (layer "F.Cu") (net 4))
 (segment (start 140.0751 76.6556) (end 144.2671 76.6556) (width 0.2) (layer "F.Cu") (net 4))
 (segment (start 126.5161 75.4826) (end 126.3131 75.6856) (width 1.5) (layer "F.Cu") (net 2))
 (segment (start 128.6151 73.385552) (end 128.6151 75.4826) (width 1.5) (layer "F.Cu") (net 2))
 (segment (start 118.9451 75.6856) (end 126.3131 75.6856) (width 1.5) (layer "F.Cu") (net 2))
 (segment (start 128.6151 75.4826) (end 128.6451 75.5126) (width 1.5) (layer "F.Cu") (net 2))
 (segment (start 128.6151 75.4826) (end 126.5161 75.4826) (width 1.5) (layer "F.Cu") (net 2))
 (segment (start 131.1551 73.385552) (end 129.028052 75.5126) (width 1.5) (layer "F.Cu") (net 2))
 (segment (start 128.6151 73.385552) (end 131.1551 73.385552) (width 1.5) (layer "F.Cu") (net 2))
 (segment (start 129.028052 75.5126) (end 128.6451 75.5126) (width 1.5) (layer "F.Cu") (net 2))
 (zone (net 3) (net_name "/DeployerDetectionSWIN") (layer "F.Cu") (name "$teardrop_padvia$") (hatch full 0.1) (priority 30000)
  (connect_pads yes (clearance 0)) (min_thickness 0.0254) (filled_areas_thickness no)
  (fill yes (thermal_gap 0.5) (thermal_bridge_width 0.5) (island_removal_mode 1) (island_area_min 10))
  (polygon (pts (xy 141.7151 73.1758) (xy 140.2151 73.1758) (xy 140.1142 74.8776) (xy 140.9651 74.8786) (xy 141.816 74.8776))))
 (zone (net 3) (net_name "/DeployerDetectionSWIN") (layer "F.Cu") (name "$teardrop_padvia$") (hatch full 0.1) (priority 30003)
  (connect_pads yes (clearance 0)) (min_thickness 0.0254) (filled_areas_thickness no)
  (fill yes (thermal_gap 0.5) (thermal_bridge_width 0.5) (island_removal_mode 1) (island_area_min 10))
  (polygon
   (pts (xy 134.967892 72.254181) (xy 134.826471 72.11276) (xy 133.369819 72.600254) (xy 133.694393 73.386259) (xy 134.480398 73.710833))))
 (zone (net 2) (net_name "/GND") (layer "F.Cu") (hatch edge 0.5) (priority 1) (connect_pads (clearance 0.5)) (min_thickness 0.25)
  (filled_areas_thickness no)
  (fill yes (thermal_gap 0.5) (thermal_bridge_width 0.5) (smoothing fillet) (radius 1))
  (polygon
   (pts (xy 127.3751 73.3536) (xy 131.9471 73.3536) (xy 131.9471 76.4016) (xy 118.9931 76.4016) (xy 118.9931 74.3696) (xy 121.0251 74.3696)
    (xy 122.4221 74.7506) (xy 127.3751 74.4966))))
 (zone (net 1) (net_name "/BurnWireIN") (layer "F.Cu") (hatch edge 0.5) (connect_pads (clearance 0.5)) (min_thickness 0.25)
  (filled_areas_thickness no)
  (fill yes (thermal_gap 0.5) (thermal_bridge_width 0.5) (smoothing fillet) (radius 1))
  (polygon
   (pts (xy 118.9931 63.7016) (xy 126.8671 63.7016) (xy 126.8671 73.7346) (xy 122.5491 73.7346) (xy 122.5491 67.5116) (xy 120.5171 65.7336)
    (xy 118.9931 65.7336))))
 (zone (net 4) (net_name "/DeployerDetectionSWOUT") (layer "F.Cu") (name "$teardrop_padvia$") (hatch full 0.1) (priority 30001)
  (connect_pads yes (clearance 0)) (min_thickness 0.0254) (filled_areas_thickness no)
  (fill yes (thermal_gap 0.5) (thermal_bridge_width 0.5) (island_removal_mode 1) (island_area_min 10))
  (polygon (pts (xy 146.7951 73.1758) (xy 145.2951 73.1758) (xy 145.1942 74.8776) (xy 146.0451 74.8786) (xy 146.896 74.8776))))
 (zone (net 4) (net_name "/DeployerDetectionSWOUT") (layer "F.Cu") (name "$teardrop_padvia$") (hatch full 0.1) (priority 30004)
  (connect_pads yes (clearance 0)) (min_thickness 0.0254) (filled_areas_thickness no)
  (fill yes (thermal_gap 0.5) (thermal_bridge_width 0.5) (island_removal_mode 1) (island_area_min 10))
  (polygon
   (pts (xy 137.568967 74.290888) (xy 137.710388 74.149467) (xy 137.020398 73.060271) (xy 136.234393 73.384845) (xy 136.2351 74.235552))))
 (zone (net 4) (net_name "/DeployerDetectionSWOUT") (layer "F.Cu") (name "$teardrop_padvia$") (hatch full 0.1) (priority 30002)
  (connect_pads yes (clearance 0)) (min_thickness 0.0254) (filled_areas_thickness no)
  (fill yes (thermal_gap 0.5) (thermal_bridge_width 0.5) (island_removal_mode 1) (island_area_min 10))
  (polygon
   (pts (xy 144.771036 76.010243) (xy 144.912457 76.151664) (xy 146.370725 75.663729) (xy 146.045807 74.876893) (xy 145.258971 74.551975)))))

